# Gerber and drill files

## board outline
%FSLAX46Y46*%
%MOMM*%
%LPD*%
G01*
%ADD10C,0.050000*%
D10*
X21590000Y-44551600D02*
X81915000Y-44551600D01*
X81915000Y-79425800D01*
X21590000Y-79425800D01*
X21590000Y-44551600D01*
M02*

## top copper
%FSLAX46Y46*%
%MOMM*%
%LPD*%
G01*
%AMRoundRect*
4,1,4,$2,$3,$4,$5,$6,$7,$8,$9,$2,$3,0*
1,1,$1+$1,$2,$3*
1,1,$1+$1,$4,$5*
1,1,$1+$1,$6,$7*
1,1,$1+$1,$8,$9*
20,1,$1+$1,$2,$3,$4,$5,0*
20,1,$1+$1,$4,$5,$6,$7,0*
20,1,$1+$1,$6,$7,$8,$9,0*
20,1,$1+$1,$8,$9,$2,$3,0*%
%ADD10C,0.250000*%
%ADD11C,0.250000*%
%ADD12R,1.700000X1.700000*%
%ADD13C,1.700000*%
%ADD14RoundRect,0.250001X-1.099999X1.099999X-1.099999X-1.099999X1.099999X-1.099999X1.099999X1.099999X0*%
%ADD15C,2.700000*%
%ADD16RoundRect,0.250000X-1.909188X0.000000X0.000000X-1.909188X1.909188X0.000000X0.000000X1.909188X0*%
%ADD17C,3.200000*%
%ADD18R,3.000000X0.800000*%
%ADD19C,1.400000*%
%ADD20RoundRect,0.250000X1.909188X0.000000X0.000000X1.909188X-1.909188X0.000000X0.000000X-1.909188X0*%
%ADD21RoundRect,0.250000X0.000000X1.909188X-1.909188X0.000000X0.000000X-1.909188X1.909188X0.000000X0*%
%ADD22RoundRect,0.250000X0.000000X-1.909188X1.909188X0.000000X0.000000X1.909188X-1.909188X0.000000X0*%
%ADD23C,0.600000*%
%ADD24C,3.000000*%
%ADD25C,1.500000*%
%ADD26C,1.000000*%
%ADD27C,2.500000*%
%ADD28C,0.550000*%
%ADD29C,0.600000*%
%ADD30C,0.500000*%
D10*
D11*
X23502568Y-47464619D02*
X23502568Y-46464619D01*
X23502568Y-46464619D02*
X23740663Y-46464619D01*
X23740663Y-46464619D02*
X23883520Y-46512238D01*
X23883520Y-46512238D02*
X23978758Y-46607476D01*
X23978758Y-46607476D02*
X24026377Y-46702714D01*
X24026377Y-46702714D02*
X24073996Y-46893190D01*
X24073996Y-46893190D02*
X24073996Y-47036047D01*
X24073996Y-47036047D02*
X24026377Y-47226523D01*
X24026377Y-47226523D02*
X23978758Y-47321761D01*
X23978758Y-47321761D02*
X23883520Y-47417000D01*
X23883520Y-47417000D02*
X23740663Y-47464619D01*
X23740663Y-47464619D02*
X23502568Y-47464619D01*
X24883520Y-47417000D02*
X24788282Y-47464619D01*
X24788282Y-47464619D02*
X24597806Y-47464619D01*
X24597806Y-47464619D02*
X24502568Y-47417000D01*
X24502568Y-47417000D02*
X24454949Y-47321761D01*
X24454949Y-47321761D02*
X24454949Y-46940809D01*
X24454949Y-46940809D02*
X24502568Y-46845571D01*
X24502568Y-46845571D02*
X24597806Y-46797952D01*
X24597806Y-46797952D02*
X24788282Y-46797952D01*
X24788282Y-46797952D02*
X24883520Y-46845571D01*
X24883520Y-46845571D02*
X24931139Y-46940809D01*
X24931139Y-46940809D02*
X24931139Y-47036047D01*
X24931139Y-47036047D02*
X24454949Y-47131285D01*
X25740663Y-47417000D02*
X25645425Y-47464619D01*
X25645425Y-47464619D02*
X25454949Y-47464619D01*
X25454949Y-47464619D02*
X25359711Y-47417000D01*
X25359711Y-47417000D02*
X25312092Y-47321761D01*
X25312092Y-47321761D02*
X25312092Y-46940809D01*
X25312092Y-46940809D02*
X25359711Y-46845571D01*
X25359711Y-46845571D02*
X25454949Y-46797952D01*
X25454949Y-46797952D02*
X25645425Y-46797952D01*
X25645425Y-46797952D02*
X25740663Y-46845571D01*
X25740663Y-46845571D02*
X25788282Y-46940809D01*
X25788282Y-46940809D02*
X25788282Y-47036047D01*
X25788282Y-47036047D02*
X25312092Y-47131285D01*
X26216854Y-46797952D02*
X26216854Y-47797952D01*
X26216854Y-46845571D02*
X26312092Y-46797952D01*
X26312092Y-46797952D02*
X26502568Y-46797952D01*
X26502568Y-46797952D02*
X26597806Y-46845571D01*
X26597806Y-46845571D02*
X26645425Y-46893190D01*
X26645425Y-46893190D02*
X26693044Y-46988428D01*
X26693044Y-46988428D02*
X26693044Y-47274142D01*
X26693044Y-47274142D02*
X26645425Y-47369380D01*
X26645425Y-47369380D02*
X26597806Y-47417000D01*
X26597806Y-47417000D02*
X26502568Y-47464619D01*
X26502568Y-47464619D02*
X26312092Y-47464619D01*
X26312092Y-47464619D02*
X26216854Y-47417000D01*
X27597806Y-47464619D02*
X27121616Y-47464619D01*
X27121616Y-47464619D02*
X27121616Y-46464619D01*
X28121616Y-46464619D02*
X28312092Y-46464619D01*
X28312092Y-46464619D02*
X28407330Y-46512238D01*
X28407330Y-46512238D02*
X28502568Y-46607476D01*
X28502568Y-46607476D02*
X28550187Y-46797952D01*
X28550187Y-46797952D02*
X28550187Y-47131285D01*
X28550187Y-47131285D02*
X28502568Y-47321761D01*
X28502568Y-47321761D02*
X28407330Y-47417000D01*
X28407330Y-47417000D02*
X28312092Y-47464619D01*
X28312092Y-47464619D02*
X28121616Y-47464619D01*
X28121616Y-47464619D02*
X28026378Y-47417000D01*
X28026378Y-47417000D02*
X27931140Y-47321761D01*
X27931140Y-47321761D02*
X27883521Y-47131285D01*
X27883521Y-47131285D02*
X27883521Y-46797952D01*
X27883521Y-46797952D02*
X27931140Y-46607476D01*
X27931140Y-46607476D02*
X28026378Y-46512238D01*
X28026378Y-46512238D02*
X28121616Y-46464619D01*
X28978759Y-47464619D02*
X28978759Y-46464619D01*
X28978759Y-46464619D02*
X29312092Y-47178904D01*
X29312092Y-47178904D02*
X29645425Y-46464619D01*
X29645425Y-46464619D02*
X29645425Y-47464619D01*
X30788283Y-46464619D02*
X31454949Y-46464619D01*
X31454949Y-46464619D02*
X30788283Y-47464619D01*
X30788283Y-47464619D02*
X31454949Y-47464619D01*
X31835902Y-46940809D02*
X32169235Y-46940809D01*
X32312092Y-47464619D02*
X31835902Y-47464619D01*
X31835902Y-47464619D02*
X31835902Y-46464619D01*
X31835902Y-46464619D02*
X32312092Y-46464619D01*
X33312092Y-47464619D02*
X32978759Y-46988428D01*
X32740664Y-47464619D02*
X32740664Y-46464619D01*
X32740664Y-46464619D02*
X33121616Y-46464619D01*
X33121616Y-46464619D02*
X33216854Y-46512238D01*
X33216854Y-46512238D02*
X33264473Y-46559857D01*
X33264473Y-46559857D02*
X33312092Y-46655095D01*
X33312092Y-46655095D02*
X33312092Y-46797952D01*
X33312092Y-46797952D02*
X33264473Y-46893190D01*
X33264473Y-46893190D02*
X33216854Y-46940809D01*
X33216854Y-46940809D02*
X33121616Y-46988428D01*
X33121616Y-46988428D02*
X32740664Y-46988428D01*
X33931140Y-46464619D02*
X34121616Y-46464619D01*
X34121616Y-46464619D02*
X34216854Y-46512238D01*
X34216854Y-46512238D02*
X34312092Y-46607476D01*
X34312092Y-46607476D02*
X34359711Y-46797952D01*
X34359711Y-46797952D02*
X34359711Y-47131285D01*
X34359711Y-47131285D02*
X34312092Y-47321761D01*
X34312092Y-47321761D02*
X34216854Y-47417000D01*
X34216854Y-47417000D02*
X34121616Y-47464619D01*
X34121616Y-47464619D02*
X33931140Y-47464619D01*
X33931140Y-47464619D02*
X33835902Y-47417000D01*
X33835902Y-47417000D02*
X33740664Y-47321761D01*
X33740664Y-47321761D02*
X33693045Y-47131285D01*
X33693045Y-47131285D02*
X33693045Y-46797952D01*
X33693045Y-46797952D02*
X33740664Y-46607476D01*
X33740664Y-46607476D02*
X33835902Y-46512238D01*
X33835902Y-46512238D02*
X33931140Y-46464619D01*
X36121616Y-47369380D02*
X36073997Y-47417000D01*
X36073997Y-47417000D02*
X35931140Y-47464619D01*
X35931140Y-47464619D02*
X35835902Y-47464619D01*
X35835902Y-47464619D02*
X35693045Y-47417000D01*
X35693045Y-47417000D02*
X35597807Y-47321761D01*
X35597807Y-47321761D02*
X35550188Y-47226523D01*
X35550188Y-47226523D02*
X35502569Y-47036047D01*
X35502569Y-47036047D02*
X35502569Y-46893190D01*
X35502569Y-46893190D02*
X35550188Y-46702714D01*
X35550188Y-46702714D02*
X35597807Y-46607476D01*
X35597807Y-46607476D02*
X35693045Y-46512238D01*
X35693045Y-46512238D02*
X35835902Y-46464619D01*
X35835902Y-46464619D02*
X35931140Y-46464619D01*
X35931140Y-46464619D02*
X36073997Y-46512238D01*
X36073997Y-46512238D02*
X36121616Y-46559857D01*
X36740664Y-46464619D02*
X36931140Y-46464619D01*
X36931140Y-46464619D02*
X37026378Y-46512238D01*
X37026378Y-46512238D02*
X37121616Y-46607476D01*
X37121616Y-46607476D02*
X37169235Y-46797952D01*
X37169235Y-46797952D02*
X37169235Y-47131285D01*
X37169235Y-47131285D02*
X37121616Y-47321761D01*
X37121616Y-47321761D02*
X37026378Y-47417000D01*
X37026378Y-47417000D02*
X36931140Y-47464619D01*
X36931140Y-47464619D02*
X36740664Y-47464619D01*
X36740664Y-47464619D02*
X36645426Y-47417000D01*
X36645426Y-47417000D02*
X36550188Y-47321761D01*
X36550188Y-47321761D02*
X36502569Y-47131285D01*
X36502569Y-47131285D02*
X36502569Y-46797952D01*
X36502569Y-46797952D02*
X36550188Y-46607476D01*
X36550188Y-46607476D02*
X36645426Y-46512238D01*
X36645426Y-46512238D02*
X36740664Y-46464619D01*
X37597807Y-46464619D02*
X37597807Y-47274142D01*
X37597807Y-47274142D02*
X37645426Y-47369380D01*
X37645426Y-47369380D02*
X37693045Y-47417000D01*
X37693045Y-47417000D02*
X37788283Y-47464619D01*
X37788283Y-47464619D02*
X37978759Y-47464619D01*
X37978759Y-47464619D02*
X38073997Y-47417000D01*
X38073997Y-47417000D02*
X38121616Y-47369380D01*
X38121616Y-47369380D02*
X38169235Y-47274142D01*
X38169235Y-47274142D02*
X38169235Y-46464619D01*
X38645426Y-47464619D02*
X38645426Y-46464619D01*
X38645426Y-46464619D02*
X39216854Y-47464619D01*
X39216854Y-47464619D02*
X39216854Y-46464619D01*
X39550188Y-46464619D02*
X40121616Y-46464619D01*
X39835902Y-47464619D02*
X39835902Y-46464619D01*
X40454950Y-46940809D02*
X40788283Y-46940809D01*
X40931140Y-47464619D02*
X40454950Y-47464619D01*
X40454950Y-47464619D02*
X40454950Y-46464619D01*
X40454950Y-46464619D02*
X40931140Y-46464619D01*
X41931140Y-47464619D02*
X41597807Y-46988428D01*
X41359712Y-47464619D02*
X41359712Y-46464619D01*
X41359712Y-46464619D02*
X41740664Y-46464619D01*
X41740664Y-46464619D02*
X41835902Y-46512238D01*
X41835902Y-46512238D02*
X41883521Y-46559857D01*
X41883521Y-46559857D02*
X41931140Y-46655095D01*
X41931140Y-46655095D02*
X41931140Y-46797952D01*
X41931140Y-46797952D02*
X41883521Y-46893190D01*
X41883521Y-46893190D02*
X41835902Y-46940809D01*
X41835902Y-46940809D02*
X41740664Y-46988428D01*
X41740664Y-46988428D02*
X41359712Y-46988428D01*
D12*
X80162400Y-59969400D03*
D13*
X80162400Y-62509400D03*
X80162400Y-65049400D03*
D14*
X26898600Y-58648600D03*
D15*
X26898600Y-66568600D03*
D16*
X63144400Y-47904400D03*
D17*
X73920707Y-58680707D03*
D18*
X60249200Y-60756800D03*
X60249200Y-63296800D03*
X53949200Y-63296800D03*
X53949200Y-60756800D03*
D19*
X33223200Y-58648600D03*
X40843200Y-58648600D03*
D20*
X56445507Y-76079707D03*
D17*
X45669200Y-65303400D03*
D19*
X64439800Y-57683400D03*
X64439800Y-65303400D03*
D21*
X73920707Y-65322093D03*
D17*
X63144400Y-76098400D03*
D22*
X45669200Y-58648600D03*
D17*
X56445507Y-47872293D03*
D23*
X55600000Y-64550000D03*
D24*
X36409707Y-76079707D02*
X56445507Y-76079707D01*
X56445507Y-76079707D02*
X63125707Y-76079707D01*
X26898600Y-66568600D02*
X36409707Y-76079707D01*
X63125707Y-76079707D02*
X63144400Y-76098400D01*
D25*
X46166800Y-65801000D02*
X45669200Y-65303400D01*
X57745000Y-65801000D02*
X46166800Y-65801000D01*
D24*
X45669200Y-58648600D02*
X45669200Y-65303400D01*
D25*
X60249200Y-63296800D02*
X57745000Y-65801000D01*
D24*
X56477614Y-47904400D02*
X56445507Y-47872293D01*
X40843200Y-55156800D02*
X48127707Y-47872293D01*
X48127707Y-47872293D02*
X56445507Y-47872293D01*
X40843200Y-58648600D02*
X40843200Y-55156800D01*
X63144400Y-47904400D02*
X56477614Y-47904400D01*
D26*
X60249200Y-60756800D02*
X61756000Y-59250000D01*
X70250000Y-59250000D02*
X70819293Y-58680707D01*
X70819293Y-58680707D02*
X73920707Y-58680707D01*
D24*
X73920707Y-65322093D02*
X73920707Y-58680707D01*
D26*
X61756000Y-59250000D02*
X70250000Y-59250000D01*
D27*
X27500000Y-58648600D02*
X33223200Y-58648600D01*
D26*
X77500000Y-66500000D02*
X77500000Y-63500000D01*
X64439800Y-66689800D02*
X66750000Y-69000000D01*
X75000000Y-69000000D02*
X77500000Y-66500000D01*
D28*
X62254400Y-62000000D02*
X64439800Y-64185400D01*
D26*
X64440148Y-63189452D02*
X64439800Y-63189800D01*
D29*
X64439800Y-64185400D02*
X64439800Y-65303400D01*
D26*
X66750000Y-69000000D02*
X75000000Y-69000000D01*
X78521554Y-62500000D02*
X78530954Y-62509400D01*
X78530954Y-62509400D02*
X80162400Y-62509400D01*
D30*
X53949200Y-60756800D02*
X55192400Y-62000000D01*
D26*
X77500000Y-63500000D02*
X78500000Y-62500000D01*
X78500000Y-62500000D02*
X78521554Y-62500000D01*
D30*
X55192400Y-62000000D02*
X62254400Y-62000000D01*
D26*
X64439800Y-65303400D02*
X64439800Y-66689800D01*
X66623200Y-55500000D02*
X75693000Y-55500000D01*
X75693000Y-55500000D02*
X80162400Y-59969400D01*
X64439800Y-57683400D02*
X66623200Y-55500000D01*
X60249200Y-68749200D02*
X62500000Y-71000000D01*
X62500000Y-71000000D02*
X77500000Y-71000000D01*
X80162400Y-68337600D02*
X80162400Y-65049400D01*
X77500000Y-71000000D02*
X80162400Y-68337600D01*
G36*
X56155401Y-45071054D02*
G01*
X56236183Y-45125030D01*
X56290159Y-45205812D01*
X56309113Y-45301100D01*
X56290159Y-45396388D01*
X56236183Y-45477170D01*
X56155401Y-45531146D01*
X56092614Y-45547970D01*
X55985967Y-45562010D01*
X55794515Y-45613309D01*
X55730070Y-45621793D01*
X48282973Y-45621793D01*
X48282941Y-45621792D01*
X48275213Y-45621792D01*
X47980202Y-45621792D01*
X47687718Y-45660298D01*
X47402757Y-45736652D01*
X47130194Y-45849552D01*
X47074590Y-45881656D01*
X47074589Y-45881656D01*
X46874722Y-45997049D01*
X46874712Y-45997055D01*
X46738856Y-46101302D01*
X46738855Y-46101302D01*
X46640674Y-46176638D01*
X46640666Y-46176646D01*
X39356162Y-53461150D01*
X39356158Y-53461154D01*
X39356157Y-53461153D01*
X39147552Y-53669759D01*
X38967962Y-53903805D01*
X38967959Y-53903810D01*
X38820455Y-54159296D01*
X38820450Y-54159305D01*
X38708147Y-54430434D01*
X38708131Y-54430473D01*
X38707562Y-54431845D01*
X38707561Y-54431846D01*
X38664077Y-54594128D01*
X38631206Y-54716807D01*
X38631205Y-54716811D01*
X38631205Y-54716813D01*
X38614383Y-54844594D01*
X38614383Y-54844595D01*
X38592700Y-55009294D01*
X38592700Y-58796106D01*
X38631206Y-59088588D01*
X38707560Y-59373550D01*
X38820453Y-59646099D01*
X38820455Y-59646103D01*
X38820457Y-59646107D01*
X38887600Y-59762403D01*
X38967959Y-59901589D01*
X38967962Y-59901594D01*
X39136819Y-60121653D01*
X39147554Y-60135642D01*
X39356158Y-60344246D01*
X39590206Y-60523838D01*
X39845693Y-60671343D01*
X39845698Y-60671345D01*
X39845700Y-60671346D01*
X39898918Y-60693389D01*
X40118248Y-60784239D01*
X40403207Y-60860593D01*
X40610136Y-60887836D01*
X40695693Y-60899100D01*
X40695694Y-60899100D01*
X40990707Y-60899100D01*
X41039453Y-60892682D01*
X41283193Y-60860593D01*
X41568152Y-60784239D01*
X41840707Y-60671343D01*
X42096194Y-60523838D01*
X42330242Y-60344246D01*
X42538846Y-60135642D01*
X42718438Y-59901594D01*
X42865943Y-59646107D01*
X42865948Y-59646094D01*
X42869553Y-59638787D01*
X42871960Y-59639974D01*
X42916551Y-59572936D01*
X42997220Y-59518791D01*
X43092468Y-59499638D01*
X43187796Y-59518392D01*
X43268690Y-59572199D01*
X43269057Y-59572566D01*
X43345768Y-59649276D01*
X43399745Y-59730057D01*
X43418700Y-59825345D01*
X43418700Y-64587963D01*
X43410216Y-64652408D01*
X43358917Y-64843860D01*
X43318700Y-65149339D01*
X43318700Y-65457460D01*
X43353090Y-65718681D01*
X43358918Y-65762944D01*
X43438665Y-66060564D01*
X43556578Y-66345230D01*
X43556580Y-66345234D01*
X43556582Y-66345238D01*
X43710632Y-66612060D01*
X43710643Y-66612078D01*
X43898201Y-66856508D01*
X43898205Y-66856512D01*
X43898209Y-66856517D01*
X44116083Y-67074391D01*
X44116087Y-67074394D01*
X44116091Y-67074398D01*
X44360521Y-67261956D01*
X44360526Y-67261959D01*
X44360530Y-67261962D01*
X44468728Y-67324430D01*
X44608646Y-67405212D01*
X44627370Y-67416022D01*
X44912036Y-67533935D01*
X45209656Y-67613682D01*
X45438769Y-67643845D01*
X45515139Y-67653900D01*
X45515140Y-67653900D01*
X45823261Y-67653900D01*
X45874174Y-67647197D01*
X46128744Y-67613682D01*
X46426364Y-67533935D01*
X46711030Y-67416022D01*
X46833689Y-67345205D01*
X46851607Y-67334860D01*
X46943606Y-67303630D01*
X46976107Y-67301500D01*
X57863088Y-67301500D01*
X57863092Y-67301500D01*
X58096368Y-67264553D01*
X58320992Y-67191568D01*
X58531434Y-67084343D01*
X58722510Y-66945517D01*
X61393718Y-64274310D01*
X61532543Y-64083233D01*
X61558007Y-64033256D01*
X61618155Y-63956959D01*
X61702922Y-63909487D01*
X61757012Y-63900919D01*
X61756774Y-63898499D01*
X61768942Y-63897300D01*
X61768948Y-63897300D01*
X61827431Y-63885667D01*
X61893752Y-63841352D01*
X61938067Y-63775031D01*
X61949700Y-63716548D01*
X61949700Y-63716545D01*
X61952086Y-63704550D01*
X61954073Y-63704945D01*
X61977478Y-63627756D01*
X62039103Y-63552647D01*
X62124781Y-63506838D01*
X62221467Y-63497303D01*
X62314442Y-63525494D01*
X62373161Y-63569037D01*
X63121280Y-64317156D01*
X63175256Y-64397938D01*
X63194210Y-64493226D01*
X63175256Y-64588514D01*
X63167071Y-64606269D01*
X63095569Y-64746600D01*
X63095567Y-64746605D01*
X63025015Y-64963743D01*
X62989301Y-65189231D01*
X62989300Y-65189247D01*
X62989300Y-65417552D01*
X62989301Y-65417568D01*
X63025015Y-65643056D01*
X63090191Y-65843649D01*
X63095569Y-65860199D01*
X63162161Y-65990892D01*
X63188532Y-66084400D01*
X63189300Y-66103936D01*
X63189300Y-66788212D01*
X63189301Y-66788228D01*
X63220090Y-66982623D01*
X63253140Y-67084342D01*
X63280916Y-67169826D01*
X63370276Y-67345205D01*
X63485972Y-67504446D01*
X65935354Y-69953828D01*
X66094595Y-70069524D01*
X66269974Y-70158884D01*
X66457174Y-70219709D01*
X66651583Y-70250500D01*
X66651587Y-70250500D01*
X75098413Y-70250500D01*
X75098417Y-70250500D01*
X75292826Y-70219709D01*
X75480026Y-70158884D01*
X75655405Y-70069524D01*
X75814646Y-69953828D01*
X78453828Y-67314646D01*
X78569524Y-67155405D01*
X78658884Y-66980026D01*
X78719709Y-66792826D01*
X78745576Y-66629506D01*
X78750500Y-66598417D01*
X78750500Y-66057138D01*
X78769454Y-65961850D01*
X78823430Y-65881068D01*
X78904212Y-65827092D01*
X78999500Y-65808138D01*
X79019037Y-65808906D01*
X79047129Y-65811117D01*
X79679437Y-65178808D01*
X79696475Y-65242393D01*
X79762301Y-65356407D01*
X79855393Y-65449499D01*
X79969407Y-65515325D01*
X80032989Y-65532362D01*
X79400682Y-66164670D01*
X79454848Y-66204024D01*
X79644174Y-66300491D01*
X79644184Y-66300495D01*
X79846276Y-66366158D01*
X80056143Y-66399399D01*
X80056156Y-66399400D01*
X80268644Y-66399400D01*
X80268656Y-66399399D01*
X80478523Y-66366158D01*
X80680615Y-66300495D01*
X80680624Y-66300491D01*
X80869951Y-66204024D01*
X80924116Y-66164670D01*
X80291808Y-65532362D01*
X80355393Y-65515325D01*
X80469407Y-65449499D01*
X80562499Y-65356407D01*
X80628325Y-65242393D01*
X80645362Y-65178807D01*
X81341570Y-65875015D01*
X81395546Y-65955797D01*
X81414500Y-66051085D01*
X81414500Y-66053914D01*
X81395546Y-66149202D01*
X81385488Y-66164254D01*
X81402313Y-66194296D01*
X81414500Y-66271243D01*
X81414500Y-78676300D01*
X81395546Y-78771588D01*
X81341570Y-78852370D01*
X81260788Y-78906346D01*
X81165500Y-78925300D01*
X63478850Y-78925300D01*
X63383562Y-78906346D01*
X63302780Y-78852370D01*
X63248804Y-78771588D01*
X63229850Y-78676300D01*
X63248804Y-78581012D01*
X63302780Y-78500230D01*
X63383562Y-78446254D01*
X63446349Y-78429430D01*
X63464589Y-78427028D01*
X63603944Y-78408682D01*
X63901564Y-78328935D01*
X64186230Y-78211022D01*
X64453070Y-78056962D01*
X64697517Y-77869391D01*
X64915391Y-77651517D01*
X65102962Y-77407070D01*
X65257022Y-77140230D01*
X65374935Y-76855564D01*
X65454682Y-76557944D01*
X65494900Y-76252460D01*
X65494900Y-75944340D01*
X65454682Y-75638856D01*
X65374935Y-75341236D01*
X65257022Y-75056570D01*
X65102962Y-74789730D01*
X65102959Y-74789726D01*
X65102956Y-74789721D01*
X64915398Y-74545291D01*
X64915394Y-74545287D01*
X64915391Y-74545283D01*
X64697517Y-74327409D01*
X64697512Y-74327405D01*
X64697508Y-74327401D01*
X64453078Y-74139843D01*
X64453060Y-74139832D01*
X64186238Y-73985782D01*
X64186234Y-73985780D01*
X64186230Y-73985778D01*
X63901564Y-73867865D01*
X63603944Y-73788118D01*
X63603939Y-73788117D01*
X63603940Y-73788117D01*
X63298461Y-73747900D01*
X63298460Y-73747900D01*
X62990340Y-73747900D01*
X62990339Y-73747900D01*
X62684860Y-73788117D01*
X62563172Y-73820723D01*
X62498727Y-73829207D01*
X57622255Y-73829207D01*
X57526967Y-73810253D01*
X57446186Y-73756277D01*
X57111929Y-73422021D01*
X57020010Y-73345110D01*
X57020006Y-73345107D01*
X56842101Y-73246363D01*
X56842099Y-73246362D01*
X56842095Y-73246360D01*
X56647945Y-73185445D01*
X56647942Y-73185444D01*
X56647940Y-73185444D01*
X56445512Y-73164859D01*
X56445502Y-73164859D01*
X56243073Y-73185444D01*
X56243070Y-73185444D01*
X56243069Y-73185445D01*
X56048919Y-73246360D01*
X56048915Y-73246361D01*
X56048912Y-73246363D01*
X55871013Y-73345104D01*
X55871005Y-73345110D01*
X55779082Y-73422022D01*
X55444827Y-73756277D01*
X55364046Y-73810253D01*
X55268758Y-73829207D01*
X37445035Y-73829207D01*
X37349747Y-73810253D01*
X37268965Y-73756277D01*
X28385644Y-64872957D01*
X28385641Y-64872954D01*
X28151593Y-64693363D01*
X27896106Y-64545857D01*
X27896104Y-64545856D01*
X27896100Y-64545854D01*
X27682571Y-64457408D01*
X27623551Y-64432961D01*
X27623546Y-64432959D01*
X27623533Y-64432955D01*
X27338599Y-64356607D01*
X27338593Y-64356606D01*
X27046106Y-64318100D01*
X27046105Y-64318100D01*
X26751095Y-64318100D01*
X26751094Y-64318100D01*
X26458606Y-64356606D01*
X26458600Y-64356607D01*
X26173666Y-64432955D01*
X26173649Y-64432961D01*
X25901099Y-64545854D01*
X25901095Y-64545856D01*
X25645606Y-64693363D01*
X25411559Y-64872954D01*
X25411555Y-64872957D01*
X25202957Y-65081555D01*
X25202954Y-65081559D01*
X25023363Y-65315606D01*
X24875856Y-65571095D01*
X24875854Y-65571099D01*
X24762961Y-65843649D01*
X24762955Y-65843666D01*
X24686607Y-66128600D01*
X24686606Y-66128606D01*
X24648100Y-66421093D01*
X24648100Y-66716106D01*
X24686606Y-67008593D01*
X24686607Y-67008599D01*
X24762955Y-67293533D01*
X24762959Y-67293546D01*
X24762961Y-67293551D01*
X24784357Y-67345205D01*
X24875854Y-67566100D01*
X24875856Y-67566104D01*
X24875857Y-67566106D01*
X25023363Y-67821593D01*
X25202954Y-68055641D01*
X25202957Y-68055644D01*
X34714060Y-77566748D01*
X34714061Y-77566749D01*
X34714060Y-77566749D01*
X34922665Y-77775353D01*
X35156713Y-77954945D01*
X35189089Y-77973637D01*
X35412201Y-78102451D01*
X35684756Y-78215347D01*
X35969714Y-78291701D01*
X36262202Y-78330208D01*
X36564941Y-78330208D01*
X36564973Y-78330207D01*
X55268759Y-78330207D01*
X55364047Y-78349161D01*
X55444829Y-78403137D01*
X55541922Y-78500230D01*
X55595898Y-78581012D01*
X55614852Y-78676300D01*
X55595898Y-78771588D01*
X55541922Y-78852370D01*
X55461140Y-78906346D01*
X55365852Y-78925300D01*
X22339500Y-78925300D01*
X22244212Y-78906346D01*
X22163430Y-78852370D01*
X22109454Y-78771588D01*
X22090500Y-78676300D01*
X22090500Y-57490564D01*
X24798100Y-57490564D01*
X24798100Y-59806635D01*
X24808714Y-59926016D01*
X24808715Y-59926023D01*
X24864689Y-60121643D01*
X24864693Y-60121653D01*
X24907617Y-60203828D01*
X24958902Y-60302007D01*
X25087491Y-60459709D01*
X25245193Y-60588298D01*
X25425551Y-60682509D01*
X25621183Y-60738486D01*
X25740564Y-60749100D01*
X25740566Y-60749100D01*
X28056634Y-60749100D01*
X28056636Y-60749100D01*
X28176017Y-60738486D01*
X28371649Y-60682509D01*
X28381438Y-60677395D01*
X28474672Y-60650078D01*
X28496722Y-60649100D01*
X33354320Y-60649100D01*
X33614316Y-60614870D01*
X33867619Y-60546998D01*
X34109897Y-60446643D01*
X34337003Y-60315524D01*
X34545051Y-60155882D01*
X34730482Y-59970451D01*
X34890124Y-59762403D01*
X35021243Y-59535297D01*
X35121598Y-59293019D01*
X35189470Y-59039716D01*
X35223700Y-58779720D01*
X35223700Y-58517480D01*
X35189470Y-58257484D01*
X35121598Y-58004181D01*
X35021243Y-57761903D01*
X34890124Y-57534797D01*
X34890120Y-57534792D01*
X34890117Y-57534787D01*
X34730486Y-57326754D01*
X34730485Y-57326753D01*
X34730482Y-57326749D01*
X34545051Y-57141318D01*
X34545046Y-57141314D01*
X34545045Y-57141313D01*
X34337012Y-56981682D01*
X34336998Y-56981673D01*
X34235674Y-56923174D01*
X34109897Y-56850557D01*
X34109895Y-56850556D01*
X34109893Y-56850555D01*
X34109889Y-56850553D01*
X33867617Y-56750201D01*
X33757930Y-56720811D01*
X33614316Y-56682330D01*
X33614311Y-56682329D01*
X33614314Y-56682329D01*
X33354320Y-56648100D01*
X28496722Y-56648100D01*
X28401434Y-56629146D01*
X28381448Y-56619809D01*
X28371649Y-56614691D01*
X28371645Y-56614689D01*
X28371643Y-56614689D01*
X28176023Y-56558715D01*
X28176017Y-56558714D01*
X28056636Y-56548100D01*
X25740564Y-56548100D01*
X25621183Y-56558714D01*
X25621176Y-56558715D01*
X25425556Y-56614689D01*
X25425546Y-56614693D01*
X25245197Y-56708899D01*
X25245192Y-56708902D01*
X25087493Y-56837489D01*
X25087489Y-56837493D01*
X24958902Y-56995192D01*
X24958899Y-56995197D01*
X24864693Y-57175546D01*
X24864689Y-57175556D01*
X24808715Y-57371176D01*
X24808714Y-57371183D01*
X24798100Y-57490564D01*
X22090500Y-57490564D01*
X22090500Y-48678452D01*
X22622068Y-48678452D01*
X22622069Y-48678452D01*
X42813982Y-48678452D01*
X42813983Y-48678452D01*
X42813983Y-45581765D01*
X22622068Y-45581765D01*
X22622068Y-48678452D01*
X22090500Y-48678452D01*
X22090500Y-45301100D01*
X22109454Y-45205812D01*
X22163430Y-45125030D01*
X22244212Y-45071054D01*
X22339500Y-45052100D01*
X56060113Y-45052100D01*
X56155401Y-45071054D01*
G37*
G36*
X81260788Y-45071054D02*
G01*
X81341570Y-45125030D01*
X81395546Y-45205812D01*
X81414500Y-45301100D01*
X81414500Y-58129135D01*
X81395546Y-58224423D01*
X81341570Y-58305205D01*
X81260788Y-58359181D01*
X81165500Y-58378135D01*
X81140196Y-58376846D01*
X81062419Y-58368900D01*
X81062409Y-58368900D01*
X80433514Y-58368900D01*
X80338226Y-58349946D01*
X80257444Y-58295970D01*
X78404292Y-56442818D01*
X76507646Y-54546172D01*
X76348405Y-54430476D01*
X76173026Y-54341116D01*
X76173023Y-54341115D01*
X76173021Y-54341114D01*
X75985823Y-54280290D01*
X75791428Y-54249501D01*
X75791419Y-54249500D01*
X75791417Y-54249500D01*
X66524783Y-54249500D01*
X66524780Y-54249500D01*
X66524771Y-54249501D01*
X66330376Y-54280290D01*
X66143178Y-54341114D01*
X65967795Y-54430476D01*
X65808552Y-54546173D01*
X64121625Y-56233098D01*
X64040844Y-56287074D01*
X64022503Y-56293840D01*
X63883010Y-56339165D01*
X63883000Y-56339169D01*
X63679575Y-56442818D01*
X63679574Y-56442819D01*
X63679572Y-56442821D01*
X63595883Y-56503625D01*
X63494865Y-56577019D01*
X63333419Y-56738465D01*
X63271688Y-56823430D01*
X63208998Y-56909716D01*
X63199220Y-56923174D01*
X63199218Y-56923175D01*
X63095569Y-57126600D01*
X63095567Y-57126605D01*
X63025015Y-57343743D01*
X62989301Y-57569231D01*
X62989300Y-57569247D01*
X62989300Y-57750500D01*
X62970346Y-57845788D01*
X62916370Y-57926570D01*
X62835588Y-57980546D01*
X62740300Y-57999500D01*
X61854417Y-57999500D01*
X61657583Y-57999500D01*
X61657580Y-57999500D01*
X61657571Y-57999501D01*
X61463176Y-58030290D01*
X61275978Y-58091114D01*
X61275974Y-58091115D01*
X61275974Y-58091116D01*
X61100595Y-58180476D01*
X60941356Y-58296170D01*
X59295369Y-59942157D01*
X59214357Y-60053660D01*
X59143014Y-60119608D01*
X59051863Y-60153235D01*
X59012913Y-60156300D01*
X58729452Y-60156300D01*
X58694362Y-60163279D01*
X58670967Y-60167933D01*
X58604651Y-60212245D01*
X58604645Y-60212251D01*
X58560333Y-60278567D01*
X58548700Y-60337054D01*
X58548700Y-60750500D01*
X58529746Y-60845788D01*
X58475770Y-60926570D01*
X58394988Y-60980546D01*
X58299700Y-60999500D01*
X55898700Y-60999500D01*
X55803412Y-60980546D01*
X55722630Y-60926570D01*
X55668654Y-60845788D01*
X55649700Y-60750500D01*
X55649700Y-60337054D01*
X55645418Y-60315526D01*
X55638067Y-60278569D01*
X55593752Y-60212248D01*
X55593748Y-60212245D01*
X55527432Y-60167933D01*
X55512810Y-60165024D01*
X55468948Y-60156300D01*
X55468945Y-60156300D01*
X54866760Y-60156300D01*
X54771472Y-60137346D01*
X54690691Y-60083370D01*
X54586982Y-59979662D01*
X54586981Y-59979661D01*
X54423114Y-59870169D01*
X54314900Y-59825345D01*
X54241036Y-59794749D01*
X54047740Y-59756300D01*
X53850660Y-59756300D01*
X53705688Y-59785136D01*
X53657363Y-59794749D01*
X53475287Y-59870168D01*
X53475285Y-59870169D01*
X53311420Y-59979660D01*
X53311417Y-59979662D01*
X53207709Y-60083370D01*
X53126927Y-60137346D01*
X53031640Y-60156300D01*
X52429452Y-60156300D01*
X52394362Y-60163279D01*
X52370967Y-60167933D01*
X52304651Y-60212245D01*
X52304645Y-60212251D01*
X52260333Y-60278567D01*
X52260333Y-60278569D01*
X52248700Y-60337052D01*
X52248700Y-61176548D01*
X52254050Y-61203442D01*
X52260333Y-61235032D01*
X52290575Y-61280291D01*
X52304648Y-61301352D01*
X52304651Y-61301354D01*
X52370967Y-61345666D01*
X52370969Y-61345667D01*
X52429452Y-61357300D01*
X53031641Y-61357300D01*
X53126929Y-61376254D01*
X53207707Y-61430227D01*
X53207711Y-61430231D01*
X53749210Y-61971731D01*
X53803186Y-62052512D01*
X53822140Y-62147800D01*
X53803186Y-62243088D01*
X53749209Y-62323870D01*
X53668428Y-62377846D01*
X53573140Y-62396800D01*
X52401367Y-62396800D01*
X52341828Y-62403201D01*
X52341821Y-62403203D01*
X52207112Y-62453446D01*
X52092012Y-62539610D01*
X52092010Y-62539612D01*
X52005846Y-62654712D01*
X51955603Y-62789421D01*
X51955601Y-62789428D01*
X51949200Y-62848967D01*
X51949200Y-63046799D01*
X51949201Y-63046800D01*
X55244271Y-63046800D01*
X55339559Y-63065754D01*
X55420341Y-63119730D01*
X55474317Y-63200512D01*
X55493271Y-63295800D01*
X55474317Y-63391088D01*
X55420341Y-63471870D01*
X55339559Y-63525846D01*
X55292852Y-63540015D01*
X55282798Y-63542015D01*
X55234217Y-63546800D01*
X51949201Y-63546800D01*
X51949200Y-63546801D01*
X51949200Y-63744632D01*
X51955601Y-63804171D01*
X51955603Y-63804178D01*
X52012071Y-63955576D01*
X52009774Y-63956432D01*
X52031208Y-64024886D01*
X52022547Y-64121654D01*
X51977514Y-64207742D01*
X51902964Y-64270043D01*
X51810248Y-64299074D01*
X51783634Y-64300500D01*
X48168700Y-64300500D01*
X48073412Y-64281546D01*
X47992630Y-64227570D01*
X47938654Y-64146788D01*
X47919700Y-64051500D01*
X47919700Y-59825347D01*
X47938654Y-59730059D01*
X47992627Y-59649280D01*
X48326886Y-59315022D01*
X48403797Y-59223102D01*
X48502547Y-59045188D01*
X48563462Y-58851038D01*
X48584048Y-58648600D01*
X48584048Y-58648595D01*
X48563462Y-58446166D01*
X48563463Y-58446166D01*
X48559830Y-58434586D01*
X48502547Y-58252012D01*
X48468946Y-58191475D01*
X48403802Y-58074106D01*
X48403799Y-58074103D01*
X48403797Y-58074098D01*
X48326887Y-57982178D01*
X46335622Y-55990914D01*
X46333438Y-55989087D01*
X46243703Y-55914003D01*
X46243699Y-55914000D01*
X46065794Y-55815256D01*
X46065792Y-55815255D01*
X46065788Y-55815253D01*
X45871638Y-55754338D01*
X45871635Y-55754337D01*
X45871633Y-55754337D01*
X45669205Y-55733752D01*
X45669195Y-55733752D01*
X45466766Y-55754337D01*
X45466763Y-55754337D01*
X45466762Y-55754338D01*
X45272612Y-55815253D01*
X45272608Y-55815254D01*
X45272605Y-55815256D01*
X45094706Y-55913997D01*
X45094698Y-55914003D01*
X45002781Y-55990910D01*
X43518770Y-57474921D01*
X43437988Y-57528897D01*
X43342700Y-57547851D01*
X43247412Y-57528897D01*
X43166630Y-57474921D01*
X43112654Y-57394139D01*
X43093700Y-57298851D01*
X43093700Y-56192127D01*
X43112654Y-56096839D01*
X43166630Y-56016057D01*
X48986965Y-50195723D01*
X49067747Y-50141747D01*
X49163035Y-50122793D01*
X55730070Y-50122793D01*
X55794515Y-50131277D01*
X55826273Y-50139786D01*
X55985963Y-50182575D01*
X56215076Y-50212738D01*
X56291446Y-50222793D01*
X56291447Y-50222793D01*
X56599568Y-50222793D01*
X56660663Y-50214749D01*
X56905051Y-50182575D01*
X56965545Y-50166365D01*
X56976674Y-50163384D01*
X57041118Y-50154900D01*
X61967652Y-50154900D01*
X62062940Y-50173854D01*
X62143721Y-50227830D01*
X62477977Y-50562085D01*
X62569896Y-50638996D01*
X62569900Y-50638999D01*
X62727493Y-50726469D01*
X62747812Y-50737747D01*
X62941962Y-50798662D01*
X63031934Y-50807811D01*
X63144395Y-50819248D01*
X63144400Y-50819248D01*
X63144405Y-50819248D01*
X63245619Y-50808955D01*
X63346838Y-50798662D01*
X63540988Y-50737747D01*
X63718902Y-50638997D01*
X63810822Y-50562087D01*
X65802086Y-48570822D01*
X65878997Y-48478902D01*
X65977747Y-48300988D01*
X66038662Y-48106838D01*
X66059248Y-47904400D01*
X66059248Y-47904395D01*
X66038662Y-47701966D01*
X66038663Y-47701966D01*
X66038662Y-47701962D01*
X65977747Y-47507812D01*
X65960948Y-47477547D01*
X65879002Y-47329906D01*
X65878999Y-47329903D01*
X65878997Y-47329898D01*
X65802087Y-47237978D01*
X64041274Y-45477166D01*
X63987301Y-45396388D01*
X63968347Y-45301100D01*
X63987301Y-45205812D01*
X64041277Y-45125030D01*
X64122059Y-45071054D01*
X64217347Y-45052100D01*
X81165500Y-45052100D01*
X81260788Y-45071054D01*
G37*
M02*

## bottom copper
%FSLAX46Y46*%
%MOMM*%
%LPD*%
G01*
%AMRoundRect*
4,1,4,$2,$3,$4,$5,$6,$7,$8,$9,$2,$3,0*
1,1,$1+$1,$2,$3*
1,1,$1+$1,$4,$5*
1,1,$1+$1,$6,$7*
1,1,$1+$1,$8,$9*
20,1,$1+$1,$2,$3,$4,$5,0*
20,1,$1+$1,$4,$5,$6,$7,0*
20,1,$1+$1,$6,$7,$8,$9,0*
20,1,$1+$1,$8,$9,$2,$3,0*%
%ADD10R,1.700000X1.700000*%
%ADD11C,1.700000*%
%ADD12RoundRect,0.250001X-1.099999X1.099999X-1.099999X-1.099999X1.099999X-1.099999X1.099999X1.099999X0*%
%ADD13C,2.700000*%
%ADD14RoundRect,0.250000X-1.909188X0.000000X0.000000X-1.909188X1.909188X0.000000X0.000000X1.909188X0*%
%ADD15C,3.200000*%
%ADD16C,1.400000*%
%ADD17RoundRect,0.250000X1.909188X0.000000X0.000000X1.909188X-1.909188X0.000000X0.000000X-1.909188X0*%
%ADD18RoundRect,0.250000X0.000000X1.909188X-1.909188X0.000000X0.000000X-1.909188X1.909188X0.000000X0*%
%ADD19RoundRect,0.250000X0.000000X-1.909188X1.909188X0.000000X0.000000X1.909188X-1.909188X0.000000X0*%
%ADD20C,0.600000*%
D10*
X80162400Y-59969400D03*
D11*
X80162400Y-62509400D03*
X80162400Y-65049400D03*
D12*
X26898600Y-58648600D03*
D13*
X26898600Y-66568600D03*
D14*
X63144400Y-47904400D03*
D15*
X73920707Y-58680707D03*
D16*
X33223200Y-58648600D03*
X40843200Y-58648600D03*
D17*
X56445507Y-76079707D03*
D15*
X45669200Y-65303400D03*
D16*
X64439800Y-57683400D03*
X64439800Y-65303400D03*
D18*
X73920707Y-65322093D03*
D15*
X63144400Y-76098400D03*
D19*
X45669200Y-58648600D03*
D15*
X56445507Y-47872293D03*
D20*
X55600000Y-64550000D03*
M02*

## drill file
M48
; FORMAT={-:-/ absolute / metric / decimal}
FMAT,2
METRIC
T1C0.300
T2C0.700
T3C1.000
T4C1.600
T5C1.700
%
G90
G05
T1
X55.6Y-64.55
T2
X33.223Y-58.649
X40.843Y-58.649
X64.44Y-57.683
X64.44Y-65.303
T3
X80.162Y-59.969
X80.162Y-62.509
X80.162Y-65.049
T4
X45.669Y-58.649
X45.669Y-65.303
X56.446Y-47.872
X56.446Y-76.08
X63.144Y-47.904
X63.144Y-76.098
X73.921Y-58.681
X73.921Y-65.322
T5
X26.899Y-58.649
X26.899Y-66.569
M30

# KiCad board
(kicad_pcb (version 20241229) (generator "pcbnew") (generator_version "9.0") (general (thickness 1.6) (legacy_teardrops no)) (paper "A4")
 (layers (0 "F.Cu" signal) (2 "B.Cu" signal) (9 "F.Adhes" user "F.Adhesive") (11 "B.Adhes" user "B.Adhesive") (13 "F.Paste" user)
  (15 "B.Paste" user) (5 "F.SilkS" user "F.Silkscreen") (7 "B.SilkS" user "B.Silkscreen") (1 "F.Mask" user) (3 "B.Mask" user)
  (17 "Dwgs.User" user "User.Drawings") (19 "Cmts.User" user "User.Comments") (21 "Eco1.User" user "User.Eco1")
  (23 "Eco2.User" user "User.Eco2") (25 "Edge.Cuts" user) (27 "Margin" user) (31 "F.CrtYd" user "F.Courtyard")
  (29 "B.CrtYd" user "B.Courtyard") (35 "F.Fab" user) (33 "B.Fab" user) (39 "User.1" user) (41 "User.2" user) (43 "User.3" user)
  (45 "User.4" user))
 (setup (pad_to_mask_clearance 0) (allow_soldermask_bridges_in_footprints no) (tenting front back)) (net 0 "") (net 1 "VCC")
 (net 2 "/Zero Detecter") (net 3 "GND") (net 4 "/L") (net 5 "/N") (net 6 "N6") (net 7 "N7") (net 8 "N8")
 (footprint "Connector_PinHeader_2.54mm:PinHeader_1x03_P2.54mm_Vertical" (layer "F.Cu") (at 80.1624 59.9694)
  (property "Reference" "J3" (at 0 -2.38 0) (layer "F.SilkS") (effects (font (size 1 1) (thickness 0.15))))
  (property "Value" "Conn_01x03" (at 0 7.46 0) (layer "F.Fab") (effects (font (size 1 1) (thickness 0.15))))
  (pad "1" thru_hole rect (at 0 0) (size 1.7 1.7) (drill 1) (layers "*.Cu" "*.Mask") (remove_unused_layers no) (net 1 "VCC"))
  (pad "2" thru_hole circle (at 0 2.54) (size 1.7 1.7) (drill 1) (layers "*.Cu" "*.Mask") (remove_unused_layers no) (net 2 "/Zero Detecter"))
  (pad "3" thru_hole circle (at 0 5.08) (size 1.7 1.7) (drill 1) (layers "*.Cu" "*.Mask") (remove_unused_layers no) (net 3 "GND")))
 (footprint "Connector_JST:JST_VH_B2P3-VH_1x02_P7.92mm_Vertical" (layer "F.Cu") (at 26.8986 58.6486 -90)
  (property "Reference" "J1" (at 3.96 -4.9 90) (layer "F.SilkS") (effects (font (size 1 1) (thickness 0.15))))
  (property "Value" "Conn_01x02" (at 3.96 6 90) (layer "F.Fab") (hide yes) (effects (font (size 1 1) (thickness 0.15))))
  (pad "1" thru_hole roundrect (at 0 0 270) (size 2.7 2.7) (drill 1.7) (layers "*.Cu" "*.Mask") (remove_unused_layers no)
   (roundrect_rratio 0.092593) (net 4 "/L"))
  (pad "2" thru_hole circle (at 7.92 0 270) (size 2.7 2.7) (drill 1.7) (layers "*.Cu" "*.Mask") (remove_unused_layers no) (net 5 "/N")))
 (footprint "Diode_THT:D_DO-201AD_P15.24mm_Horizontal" (layer "F.Cu") (at 63.1444 47.9044 -45)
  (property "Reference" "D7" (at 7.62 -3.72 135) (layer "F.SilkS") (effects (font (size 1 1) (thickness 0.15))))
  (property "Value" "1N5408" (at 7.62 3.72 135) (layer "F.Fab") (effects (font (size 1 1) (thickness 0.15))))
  (pad "1" thru_hole roundrect (at 0 0 315) (size 3.2 3.2) (drill 1.6) (layers "*.Cu" "*.Mask") (remove_unused_layers no)
   (roundrect_rratio 0.078125) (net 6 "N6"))
  (pad "2" thru_hole circle (at 15.24 0 315) (size 3.2 3.2) (drill 1.6) (layers "*.Cu" "*.Mask") (remove_unused_layers no) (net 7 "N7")))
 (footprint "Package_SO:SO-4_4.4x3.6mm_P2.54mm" (layer "F.Cu") (at 57.0992 62.0268)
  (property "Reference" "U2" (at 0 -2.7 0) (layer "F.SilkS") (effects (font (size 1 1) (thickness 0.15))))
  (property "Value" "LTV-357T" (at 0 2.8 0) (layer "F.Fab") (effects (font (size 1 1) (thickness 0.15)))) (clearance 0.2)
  (pad "1" smd rect (at 3.15 -1.27) (size 3 0.8) (layers "F.Cu" "F.Mask" "F.Paste") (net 7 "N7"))
  (pad "2" smd rect (at 3.15 1.27) (size 3 0.8) (layers "F.Cu" "F.Mask" "F.Paste") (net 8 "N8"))
  (pad "3" smd rect (at -3.15 1.27) (size 3 0.8) (layers "F.Cu" "F.Mask" "F.Paste") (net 3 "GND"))
  (pad "4" smd rect (at -3.15 -1.27) (size 3 0.8) (layers "F.Cu" "F.Mask" "F.Paste") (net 2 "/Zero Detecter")))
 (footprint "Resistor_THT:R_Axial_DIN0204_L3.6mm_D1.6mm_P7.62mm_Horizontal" (layer "F.Cu") (at 33.2232 58.6486)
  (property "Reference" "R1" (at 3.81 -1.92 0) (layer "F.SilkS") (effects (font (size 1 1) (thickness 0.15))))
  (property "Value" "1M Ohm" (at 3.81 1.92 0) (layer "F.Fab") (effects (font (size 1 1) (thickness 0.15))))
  (pad "1" thru_hole circle (at 0 0) (size 1.4 1.4) (drill 0.7) (layers "*.Cu" "*.Mask") (remove_unused_layers no) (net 4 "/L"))
  (pad "2" thru_hole circle (at 7.62 0) (size 1.4 1.4) (drill 0.7) (layers "*.Cu" "*.Mask") (remove_unused_layers no) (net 6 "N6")))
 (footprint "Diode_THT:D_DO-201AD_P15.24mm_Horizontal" (layer "F.Cu") (at 56.445507 76.079707 135)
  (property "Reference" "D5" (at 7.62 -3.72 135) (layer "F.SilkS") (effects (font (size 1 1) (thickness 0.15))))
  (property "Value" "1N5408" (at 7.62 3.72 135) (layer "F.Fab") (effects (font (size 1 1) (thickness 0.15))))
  (pad "1" thru_hole roundrect (at 0 0 135) (size 3.2 3.2) (drill 1.6) (layers "*.Cu" "*.Mask") (remove_unused_layers no)
   (roundrect_rratio 0.078125) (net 5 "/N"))
  (pad "2" thru_hole circle (at 15.24 0 135) (size 3.2 3.2) (drill 1.6) (layers "*.Cu" "*.Mask") (remove_unused_layers no) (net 8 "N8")))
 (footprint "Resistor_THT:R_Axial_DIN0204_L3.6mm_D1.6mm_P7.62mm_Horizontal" (layer "F.Cu") (at 64.4398 57.6834 -90)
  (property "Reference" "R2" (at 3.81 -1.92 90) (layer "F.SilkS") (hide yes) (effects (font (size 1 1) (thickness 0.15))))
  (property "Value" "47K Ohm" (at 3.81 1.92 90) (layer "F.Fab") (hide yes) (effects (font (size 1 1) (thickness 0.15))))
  (pad "1" thru_hole circle (at 0 0 270) (size 1.4 1.4) (drill 0.7) (layers "*.Cu" "*.Mask") (remove_unused_layers no) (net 1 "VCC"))
  (pad "2" thru_hole circle (at 7.62 0 270) (size 1.4 1.4) (drill 0.7) (layers "*.Cu" "*.Mask") (remove_unused_layers no)
   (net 2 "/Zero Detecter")))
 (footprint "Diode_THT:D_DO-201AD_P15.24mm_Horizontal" (layer "F.Cu") (at 73.920707 65.322093 -135)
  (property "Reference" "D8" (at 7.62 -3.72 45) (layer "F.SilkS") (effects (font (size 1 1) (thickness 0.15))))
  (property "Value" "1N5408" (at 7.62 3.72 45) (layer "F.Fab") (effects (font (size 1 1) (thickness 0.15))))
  (pad "1" thru_hole roundrect (at 0 0 225) (size 3.2 3.2) (drill 1.6) (layers "*.Cu" "*.Mask") (remove_unused_layers no)
   (roundrect_rratio 0.078125) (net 7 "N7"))
  (pad "2" thru_hole circle (at 15.24 0 225) (size 3.2 3.2) (drill 1.6) (layers "*.Cu" "*.Mask") (remove_unused_layers no) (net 5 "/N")))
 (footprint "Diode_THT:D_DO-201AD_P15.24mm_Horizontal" (layer "F.Cu") (at 45.6692 58.6486 45)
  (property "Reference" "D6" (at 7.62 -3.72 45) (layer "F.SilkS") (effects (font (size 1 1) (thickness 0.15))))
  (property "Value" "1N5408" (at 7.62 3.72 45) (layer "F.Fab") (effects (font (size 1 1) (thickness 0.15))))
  (pad "1" thru_hole roundrect (at 0 0 45) (size 3.2 3.2) (drill 1.6) (layers "*.Cu" "*.Mask") (remove_unused_layers no)
   (roundrect_rratio 0.078125) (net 8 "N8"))
  (pad "2" thru_hole circle (at 15.24 0 45) (size 3.2 3.2) (drill 1.6) (layers "*.Cu" "*.Mask") (remove_unused_layers no) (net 6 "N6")))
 (gr_rect (start 21.59 44.5516) (end 81.915 79.4258) (stroke (width 0.05) (type default)) (fill no) (layer "Edge.Cuts"))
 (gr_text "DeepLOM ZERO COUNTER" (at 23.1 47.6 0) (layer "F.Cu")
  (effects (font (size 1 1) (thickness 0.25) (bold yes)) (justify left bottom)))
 (via (at 55.6 64.55) (size 0.6) (drill 0.3) (layers "F.Cu" "B.Cu") (free yes) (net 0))
 (segment (start 36.409707 76.079707) (end 56.445507 76.079707) (width 3) (layer "F.Cu") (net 5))
 (segment (start 56.445507 76.079707) (end 63.125707 76.079707) (width 3) (layer "F.Cu") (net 5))
 (segment (start 26.8986 66.5686) (end 36.409707 76.079707) (width 3) (layer "F.Cu") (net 5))
 (segment (start 63.125707 76.079707) (end 63.1444 76.0984) (width 3) (layer "F.Cu") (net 5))
 (segment (start 46.1668 65.801) (end 45.6692 65.3034) (width 1.5) (layer "F.Cu") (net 8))
 (segment (start 57.745 65.801) (end 46.1668 65.801) (width 1.5) (layer "F.Cu") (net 8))
 (segment (start 45.6692 58.6486) (end 45.6692 65.3034) (width 3) (layer "F.Cu") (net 8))
 (segment (start 60.2492 63.2968) (end 57.745 65.801) (width 1.5) (layer "F.Cu") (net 8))
 (segment (start 56.477614 47.9044) (end 56.445507 47.872293) (width 3) (layer "F.Cu") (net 6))
 (segment (start 40.8432 55.1568) (end 48.127707 47.872293) (width 3) (layer "F.Cu") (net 6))
 (segment (start 48.127707 47.872293) (end 56.445507 47.872293) (width 3) (layer "F.Cu") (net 6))
 (segment (start 40.8432 58.6486) (end 40.8432 55.1568) (width 3) (layer "F.Cu") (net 6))
 (segment (start 63.1444 47.9044) (end 56.477614 47.9044) (width 3) (layer "F.Cu") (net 6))
 (segment (start 60.2492 60.7568) (end 61.756 59.25) (width 1) (layer "F.Cu") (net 7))
 (segment (start 70.25 59.25) (end 70.819293 58.680707) (width 1) (layer "F.Cu") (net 7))
 (segment (start 70.819293 58.680707) (end 73.920707 58.680707) (width 1) (layer "F.Cu") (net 7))
 (segment (start 73.920707 65.322093) (end 73.920707 58.680707) (width 3) (layer "F.Cu") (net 7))
 (segment (start 61.756 59.25) (end 70.25 59.25) (width 1) (layer "F.Cu") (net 7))
 (segment (start 27.5 58.6486) (end 33.2232 58.6486) (width 2.5) (layer "F.Cu") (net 4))
 (segment (start 77.5 66.5) (end 77.5 63.5) (width 1) (layer "F.Cu") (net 2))
 (segment (start 64.4398 66.6898) (end 66.75 69) (width 1) (layer "F.Cu") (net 2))
 (segment (start 75 69) (end 77.5 66.5) (width 1) (layer "F.Cu") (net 2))
 (segment (start 62.2544 62) (end 64.4398 64.1854) (width 0.55) (layer "F.Cu") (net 2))
 (segment (start 64.440148 63.189452) (end 64.4398 63.1898) (width 1) (layer "F.Cu") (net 2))
 (segment (start 64.4398 64.1854) (end 64.4398 65.3034) (width 0.6) (layer "F.Cu") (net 2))
 (segment (start 66.75 69) (end 75 69) (width 1) (layer "F.Cu") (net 2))
 (segment (start 78.521554 62.5) (end 78.530954 62.5094) (width 1) (layer "F.Cu") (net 2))
 (segment (start 78.530954 62.5094) (end 80.1624 62.5094) (width 1) (layer "F.Cu") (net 2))
 (segment (start 53.9492 60.7568) (end 55.1924 62) (width 0.5) (layer "F.Cu") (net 2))
 (segment (start 77.5 63.5) (end 78.5 62.5) (width 1) (layer "F.Cu") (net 2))
 (segment (start 78.5 62.5) (end 78.521554 62.5) (width 1) (layer "F.Cu") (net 2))
 (segment (start 55.1924 62) (end 62.2544 62) (width 0.5) (layer "F.Cu") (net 2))
 (segment (start 64.4398 65.3034) (end 64.4398 66.6898) (width 1) (layer "F.Cu") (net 2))
 (segment (start 66.6232 55.5) (end 75.693 55.5) (width 1) (layer "F.Cu") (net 1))
 (segment (start 75.693 55.5) (end 80.1624 59.9694) (width 1) (layer "F.Cu") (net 1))
 (segment (start 64.4398 57.6834) (end 66.6232 55.5) (width 1) (layer "F.Cu") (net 1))
 (segment (start 60.2492 68.7492) (end 62.5 71) (width 1) (layer "F.Cu") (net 3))
 (segment (start 62.5 71) (end 77.5 71) (width 1) (layer "F.Cu") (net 3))
 (segment (start 80.1624 68.3376) (end 80.1624 65.0494) (width 1) (layer "F.Cu") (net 3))
 (segment (start 77.5 71) (end 80.1624 68.3376) (width 1) (layer "F.Cu") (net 3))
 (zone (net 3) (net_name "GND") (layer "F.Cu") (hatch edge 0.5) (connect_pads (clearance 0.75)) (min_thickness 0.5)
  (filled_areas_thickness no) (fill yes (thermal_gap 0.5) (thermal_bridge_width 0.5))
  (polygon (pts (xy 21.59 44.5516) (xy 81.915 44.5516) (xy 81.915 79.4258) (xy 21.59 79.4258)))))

